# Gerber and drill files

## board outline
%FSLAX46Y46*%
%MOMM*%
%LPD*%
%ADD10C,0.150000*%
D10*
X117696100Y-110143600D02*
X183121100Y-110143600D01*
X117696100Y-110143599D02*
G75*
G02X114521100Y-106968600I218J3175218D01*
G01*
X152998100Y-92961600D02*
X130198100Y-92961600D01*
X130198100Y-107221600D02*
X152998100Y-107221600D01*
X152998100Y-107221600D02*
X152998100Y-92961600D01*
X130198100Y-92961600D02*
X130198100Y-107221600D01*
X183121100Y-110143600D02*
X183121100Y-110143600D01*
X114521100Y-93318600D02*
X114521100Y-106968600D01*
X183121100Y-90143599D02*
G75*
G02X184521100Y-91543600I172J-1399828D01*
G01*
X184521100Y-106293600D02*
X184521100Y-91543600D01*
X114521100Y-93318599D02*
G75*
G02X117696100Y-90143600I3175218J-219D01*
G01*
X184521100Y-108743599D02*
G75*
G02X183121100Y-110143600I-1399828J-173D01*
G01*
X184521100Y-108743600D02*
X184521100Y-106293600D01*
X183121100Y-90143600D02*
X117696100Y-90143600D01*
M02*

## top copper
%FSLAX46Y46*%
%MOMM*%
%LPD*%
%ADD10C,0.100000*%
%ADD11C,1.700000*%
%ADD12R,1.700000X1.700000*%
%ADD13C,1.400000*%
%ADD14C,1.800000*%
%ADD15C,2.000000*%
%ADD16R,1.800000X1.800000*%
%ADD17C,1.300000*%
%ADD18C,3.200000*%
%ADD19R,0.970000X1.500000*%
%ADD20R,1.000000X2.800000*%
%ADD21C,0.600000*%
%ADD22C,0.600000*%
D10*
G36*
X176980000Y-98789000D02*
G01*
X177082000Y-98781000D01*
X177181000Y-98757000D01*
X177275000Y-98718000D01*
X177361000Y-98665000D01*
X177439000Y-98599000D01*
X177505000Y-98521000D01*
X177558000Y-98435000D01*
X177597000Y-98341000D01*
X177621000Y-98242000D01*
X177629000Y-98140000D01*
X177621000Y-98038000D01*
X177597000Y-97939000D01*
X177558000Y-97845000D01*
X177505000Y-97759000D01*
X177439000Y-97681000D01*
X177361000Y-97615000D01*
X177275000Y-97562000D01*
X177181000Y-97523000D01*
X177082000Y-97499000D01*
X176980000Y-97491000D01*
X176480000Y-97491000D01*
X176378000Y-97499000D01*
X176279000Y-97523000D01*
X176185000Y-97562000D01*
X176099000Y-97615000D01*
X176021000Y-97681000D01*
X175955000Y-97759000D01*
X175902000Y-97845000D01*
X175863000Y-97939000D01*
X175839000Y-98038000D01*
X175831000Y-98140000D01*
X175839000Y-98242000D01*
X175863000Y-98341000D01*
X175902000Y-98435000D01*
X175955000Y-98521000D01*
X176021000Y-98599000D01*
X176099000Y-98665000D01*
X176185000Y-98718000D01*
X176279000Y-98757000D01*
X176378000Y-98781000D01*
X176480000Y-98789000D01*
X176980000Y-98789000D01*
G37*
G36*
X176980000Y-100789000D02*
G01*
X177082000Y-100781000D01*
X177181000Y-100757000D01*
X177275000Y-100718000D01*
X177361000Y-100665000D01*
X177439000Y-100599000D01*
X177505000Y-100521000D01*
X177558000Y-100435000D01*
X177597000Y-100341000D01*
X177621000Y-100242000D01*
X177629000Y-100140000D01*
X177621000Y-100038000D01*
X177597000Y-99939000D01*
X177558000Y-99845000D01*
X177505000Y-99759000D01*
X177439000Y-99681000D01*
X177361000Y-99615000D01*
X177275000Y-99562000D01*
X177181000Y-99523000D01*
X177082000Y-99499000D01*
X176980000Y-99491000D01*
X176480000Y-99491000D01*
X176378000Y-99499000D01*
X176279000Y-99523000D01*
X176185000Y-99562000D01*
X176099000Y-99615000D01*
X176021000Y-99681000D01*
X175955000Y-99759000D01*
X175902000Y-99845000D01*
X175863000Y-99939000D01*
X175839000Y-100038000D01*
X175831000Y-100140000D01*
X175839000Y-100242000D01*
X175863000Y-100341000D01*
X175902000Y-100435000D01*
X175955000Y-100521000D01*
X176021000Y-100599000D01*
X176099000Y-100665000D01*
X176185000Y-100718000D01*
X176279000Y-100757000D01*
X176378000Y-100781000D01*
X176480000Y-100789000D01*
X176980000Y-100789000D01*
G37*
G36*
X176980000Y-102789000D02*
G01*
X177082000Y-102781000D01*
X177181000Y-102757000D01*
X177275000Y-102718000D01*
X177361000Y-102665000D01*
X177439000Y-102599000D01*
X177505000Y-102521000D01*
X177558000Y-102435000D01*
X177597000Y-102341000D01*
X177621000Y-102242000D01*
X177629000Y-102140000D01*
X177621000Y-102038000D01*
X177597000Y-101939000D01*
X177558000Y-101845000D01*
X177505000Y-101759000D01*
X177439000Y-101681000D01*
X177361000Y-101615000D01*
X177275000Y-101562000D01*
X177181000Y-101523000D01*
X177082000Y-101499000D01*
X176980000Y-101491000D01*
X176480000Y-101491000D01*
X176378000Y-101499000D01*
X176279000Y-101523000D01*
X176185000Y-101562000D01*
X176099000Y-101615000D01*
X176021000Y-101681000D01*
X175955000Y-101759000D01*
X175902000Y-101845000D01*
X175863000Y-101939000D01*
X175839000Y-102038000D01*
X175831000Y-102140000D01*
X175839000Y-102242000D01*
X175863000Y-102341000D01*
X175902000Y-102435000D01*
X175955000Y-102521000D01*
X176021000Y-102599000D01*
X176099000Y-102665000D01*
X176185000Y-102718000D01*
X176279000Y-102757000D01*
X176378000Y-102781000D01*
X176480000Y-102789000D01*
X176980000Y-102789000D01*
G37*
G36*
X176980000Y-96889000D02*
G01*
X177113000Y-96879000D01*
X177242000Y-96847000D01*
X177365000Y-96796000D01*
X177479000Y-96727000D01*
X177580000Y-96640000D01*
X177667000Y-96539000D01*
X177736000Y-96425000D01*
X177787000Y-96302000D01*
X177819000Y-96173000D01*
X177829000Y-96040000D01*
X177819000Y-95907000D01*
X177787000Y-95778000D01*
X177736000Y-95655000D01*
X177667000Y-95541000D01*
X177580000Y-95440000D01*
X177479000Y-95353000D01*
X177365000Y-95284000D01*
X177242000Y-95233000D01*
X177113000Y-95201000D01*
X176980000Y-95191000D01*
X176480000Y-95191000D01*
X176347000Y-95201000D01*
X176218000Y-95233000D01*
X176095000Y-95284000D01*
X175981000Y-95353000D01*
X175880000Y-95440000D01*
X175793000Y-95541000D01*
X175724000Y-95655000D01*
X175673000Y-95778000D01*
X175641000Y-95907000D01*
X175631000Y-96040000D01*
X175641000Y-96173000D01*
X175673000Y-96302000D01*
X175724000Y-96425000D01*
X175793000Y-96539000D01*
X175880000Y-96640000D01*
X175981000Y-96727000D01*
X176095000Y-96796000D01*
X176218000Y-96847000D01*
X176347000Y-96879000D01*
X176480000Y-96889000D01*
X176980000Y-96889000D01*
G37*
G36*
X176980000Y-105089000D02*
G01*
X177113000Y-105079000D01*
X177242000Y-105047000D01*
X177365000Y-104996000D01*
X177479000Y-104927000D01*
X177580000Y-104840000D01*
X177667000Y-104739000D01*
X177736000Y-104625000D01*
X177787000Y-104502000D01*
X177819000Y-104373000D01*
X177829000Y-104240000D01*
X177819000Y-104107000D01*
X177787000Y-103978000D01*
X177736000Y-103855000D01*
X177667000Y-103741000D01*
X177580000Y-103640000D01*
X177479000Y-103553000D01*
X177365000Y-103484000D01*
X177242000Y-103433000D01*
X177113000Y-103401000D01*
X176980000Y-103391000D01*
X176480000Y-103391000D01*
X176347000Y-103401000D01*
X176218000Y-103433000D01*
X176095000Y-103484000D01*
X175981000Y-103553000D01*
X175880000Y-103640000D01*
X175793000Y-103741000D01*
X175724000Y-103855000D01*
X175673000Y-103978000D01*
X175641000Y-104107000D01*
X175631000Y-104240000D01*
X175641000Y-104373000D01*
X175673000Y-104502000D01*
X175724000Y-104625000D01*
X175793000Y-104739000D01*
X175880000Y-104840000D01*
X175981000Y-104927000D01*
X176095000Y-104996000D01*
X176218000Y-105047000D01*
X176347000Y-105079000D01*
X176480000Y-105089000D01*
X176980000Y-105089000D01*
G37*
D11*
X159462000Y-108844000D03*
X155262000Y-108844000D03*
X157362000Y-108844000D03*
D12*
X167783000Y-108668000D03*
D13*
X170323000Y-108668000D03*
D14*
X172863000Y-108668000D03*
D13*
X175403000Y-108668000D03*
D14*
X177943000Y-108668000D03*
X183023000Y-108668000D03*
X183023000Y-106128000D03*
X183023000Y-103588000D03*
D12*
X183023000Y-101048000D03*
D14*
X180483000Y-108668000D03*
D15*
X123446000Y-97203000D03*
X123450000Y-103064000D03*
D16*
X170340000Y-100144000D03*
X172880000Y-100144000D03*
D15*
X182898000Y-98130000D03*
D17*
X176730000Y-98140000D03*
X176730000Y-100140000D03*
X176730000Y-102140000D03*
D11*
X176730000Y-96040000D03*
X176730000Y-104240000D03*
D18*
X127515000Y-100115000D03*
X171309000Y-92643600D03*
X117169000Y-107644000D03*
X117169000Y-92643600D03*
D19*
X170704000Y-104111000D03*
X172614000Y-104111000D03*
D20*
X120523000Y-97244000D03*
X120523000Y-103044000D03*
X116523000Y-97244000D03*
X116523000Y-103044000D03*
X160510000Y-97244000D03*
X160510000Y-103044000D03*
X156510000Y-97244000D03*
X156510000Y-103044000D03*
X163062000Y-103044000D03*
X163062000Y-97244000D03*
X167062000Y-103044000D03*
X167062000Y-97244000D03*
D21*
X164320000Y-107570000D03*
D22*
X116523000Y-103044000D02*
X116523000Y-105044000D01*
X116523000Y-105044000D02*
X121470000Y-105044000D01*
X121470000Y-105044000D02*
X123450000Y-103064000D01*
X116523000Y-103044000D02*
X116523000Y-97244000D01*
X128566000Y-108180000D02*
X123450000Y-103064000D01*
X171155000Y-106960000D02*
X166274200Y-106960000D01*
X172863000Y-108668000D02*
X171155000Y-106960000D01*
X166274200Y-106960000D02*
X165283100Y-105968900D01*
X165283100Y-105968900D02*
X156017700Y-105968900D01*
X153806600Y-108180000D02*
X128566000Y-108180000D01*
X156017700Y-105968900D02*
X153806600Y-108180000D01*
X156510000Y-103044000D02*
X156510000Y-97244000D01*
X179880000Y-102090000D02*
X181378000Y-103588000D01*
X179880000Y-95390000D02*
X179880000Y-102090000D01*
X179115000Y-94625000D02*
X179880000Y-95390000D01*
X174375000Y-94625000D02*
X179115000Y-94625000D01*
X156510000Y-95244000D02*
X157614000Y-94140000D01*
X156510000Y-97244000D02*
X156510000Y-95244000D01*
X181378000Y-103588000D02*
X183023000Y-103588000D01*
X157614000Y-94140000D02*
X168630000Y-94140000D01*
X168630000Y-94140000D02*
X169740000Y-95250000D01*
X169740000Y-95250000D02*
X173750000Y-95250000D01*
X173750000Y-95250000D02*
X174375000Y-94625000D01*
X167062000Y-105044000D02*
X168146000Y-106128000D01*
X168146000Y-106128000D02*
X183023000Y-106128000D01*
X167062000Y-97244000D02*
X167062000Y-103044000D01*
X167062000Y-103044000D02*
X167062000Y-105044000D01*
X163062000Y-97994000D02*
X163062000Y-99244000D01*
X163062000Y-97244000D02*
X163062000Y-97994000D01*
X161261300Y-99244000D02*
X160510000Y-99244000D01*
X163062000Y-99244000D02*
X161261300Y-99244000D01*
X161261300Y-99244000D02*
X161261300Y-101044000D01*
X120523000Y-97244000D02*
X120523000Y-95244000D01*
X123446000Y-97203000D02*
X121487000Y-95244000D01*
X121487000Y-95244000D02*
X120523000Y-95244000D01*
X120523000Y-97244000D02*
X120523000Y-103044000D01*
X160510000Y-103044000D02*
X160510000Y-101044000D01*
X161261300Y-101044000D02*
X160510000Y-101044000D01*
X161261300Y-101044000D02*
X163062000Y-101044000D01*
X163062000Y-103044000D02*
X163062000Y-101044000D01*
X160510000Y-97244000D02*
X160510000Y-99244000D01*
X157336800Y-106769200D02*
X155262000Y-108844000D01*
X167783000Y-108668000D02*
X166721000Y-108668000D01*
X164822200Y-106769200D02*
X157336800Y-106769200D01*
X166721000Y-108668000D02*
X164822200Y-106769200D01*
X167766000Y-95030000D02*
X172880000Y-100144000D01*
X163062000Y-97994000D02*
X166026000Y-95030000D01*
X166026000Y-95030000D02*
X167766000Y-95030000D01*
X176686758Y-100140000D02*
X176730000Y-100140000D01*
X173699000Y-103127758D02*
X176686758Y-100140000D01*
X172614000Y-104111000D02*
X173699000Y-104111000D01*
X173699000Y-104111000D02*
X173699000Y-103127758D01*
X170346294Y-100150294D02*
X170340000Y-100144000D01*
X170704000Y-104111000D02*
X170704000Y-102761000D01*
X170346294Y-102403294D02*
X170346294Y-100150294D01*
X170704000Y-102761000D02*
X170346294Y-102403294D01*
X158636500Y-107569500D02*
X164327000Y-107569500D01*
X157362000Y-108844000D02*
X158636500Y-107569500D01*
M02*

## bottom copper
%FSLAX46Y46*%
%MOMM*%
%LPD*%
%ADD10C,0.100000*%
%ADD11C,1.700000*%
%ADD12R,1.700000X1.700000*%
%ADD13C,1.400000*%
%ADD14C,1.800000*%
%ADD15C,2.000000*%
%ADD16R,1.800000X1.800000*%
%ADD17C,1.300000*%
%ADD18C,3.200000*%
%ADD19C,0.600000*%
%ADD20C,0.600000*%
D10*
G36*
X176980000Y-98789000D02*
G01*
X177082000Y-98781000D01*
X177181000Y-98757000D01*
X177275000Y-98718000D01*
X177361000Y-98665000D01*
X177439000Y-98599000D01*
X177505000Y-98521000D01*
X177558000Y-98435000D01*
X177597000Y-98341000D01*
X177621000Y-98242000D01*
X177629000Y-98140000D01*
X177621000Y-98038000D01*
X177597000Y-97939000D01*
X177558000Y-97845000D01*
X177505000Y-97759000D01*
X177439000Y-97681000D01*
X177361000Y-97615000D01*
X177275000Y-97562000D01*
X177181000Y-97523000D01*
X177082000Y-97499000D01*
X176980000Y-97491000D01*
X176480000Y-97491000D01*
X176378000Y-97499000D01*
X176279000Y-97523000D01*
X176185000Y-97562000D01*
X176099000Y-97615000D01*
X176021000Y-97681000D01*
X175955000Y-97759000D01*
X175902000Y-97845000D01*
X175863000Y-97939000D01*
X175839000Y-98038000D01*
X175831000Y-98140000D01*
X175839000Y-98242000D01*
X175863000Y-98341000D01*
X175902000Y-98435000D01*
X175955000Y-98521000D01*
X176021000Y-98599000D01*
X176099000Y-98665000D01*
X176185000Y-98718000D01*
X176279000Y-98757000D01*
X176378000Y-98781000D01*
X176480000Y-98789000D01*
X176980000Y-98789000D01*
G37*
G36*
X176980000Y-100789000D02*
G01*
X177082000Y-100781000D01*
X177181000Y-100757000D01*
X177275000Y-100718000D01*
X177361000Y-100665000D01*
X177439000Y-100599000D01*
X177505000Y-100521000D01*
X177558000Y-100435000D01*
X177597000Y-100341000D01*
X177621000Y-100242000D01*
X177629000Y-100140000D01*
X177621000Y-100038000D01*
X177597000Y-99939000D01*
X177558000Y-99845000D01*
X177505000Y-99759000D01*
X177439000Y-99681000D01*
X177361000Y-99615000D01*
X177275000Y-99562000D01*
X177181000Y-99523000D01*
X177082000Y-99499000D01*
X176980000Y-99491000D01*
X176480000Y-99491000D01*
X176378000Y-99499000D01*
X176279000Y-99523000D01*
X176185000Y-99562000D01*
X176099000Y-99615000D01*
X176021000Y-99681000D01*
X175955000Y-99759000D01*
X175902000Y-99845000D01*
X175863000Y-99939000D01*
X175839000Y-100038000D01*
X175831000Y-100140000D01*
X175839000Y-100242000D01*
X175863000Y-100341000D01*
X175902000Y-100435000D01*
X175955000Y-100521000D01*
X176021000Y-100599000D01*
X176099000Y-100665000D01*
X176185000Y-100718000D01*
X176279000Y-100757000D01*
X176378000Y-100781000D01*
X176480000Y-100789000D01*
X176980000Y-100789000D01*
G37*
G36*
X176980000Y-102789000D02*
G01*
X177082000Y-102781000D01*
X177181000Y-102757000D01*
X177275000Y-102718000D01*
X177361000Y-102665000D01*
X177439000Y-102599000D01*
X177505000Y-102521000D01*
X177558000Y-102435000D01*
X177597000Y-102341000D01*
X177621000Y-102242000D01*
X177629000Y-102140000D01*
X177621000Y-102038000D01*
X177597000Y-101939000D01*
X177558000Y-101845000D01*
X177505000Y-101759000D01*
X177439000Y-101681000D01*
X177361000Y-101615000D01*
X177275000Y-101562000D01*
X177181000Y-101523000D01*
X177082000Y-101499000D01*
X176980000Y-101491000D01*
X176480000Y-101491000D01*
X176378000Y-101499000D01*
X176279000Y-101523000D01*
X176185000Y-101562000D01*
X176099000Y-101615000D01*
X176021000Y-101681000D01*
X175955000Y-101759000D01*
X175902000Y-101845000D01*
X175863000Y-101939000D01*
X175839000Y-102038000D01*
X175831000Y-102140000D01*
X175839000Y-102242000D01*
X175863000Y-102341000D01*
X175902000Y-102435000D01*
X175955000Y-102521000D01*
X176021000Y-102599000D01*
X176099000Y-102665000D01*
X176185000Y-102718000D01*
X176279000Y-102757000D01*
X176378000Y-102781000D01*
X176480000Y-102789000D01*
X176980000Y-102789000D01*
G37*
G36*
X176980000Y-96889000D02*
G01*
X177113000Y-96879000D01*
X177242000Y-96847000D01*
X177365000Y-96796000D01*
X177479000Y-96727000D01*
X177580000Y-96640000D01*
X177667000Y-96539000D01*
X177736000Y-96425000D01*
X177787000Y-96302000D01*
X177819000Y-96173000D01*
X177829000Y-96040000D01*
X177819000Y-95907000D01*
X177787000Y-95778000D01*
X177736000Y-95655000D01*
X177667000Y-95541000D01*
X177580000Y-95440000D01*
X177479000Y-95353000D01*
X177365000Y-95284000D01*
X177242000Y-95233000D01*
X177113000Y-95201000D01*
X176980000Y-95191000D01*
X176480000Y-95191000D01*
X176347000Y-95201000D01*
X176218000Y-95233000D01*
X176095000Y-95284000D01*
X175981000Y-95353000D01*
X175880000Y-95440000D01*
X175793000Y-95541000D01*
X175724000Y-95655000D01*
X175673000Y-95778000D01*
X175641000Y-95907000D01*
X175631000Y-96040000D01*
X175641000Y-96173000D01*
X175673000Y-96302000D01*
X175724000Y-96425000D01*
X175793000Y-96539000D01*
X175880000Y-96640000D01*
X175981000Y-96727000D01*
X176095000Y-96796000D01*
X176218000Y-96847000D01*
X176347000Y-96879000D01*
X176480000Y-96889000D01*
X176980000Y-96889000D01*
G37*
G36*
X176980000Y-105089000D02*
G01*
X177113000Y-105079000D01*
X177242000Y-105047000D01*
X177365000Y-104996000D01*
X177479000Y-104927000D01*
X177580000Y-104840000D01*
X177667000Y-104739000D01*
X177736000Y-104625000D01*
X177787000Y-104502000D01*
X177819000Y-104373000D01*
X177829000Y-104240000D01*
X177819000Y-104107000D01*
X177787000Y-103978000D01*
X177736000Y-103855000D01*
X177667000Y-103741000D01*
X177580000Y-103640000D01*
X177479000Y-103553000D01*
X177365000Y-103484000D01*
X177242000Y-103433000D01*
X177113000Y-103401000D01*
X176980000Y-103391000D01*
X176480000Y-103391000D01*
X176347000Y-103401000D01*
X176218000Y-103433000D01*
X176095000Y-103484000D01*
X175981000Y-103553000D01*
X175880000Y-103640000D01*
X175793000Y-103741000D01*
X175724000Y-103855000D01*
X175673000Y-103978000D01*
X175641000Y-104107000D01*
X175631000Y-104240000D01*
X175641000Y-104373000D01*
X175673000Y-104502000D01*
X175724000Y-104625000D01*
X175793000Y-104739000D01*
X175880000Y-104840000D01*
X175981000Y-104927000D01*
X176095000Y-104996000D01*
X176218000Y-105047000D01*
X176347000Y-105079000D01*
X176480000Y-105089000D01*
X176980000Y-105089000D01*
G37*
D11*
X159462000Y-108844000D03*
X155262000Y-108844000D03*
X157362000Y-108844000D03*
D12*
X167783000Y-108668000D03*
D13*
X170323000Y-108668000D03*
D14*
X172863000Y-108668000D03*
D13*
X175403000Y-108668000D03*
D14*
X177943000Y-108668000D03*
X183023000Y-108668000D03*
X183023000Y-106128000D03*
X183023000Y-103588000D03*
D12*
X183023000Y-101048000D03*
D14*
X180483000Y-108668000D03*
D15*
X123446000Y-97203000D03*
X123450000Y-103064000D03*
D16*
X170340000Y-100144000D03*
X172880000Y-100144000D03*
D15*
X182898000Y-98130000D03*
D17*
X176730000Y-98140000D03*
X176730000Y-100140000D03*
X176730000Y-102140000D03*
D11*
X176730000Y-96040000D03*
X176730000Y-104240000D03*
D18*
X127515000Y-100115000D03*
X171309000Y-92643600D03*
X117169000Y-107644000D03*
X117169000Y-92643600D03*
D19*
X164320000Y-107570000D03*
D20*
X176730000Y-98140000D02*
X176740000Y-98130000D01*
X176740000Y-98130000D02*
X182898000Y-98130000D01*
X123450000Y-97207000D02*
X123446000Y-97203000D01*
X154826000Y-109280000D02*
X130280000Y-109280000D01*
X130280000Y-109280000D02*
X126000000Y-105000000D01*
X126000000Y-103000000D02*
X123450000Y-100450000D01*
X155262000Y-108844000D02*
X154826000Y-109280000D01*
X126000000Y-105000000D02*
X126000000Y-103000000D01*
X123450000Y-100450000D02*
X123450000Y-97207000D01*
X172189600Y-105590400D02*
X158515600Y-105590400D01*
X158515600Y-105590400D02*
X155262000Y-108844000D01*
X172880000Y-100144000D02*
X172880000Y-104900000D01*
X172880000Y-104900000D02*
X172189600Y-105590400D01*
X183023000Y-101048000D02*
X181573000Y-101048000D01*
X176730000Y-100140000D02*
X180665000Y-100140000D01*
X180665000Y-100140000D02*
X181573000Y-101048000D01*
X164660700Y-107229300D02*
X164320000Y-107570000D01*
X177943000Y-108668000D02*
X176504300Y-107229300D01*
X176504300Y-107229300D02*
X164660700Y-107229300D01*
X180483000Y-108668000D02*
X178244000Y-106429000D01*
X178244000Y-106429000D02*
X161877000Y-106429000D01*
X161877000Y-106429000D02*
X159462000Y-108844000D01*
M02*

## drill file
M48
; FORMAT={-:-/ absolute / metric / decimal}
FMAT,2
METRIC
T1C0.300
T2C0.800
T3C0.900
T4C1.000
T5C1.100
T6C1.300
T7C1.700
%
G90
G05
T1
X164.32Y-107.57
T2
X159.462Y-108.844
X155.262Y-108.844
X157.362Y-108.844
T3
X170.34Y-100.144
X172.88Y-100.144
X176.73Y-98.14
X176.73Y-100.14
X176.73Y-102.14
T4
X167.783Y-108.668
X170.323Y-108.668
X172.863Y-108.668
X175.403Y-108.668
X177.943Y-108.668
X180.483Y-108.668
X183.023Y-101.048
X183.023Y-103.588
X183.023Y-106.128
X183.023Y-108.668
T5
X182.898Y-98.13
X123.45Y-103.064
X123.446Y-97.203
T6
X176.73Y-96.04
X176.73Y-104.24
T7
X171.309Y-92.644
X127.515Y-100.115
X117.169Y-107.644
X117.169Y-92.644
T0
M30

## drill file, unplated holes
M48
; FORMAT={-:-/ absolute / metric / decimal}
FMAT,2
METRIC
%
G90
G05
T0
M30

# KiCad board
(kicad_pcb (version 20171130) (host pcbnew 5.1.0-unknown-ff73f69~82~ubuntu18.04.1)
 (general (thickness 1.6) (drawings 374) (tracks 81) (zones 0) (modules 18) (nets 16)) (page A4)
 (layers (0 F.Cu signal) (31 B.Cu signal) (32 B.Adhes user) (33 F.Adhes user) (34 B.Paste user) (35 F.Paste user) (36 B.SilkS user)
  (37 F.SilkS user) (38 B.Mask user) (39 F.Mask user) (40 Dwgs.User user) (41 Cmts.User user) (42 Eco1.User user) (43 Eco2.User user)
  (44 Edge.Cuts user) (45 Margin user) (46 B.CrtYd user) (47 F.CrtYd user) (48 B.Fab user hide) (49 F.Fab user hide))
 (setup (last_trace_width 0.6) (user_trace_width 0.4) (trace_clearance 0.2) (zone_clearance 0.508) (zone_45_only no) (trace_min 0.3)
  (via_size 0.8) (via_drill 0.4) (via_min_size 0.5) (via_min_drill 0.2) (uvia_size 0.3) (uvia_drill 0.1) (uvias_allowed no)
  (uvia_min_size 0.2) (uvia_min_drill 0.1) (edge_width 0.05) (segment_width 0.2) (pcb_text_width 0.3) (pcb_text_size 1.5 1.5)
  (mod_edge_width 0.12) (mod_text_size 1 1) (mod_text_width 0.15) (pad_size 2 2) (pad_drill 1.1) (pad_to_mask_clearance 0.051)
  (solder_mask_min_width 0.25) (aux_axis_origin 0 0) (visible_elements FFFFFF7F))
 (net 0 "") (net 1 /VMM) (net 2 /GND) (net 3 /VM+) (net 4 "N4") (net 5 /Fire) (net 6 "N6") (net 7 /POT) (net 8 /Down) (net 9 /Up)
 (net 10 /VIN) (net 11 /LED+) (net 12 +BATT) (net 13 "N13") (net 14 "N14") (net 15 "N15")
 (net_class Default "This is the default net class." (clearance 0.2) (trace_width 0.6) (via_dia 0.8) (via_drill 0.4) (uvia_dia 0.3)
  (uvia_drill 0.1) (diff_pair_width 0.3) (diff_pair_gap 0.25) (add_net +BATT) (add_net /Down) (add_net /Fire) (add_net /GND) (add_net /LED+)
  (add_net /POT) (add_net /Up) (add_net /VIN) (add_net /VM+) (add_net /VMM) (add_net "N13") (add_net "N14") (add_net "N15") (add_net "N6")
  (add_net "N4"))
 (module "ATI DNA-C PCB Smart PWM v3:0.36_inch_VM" (layer F.Cu) (at 141.72 100.27)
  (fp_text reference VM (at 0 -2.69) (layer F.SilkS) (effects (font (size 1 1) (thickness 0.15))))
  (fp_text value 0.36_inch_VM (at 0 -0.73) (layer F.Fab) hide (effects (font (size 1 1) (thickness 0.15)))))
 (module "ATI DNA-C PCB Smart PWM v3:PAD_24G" (layer F.Cu) (at 159.462 108.844)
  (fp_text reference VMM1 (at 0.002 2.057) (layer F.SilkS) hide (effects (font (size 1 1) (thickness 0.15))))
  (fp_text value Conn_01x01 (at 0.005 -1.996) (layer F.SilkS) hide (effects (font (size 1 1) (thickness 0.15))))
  (pad 1 thru_hole circle (at 0 0 90) (size 1.7 1.7) (drill 0.8) (layers *.Cu *.Mask) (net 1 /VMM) (solder_mask_margin 0.1016)
   (zone_connect 2)))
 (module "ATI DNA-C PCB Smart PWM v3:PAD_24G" (layer F.Cu) (at 155.262 108.844)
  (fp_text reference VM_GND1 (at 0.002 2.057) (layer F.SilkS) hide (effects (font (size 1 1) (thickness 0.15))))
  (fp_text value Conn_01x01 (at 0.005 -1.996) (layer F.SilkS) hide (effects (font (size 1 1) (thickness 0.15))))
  (pad 1 thru_hole circle (at 0 0 90) (size 1.7 1.7) (drill 0.8) (layers *.Cu *.Mask) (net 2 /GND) (solder_mask_margin 0.1016)
   (zone_connect 2)))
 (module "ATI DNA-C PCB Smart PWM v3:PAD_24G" (layer F.Cu) (at 157.362 108.844)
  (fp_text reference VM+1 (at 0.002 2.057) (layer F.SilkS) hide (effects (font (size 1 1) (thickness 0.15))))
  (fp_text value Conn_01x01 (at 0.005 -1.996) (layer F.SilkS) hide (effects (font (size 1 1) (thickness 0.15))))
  (pad 1 thru_hole circle (at 0 0 90) (size 1.7 1.7) (drill 0.8) (layers *.Cu *.Mask) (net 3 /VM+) (solder_mask_margin 0.1016)
   (zone_connect 2)))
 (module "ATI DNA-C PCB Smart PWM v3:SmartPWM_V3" (layer F.Cu) (at 175.438 104.848)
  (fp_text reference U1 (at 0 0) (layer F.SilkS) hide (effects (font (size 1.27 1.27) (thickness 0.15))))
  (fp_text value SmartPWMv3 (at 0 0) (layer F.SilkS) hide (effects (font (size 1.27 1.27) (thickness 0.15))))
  (pad 10 thru_hole rect (at -7.655 3.82) (size 1.7 1.7) (drill 1) (layers *.Cu *.Mask) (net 2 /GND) (zone_connect 2))
  (pad 9 thru_hole circle (at -5.115 3.82) (size 1.4 1.4) (drill 1) (layers *.Cu *.Mask) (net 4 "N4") (zone_connect 2))
  (pad 8 thru_hole circle (at -2.575 3.82) (size 1.8 1.8) (drill 1) (layers *.Cu *.Mask) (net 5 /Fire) (zone_connect 2))
  (pad 7 thru_hole circle (at -0.035 3.82) (size 1.4 1.4) (drill 1) (layers *.Cu *.Mask) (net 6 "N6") (zone_connect 2))
  (pad 6 thru_hole circle (at 2.505 3.82) (size 1.8 1.8) (drill 1) (layers *.Cu *.Mask) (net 3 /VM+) (zone_connect 2))
  (pad 4 thru_hole circle (at 7.585 3.82) (size 1.8 1.8) (drill 1) (layers *.Cu *.Mask) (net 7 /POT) (zone_connect 2))
  (pad 3 thru_hole circle (at 7.585 1.28) (size 1.8 1.8) (drill 1) (layers *.Cu *.Mask) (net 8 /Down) (zone_connect 2))
  (pad 2 thru_hole circle (at 7.585 -1.26) (size 1.8 1.8) (drill 1) (layers *.Cu *.Mask) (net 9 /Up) (zone_connect 2))
  (pad 1 thru_hole rect (at 7.585 -3.8 90) (size 1.7 1.7) (drill 1) (layers *.Cu *.Mask) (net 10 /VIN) (zone_connect 2))
  (pad 5 thru_hole circle (at 5.045 3.82) (size 1.8 1.8) (drill 1) (layers *.Cu *.Mask) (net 1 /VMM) (zone_connect 2)))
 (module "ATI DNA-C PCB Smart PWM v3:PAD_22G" (layer F.Cu) (at 123.446 97.203)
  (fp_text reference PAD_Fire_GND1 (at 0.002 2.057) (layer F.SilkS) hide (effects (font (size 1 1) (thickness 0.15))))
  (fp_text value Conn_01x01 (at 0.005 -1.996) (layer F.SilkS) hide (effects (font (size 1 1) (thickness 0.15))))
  (pad 1 thru_hole circle (at 0 0 90) (size 2 2) (drill 1.1) (layers *.Cu *.Mask) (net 2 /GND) (solder_mask_margin 0.1016) (zone_connect 2)))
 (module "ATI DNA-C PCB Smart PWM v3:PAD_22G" (layer F.Cu) (at 123.45 103.064)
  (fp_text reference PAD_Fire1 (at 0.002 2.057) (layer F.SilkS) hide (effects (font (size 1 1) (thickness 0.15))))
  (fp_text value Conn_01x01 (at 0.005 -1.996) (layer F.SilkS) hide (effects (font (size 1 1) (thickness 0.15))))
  (pad 1 thru_hole circle (at 0 0 90) (size 2 2) (drill 1.1) (layers *.Cu *.Mask) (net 5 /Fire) (solder_mask_margin 0.1016) (zone_connect 2)))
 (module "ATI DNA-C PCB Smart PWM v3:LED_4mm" (layer F.Cu) (at 171.62 100.144 180)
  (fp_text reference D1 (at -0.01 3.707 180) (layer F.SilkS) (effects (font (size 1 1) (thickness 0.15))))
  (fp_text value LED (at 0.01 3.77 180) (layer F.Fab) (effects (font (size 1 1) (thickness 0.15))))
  (pad 2 thru_hole rect (at 1.28 0 180) (size 1.8 1.8) (drill 0.9) (layers *.Cu *.Mask) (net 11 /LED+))
  (pad 1 thru_hole rect (at -1.26 0 180) (size 1.8 1.8) (drill 0.9) (layers *.Cu *.Mask) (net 2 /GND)))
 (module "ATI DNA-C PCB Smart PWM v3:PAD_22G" (layer F.Cu) (at 182.898 98.13)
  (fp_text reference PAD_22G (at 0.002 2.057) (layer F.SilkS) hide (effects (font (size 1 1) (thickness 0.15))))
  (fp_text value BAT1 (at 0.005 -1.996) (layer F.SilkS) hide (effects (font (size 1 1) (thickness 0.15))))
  (pad 1 thru_hole circle (at 0 0 90) (size 2 2) (drill 1.1) (layers *.Cu *.Mask) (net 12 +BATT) (solder_mask_margin 0.1016)
   (zone_connect 2)))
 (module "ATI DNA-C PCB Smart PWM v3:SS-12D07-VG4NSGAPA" (layer F.Cu) (at 176.73 100.14 270)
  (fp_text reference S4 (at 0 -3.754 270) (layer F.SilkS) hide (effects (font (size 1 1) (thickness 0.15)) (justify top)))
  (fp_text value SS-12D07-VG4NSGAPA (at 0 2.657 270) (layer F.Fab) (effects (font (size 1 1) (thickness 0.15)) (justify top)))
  (fp_poly
   (pts (xy -1.351 -0.25) (xy -1.359 -0.352) (xy -1.383 -0.451) (xy -1.422 -0.545) (xy -1.475 -0.631) (xy -1.541 -0.709) (xy -1.619 -0.775)
    (xy -1.705 -0.828) (xy -1.799 -0.867) (xy -1.898 -0.891) (xy -2 -0.899) (xy -2.102 -0.891) (xy -2.201 -0.867) (xy -2.295 -0.828)
    (xy -2.381 -0.775) (xy -2.459 -0.709) (xy -2.525 -0.631) (xy -2.578 -0.545) (xy -2.617 -0.451) (xy -2.641 -0.352) (xy -2.649 -0.25)
    (xy -2.649 0.25) (xy -2.641 0.352) (xy -2.617 0.451) (xy -2.578 0.545) (xy -2.525 0.631) (xy -2.459 0.709) (xy -2.381 0.775)
    (xy -2.295 0.828) (xy -2.201 0.867) (xy -2.102 0.891) (xy -2 0.899) (xy -1.898 0.891) (xy -1.799 0.867) (xy -1.705 0.828)
    (xy -1.619 0.775) (xy -1.541 0.709) (xy -1.475 0.631) (xy -1.422 0.545) (xy -1.383 0.451) (xy -1.359 0.352) (xy -1.351 0.25))
   (layer F.Cu) (width 0))
  (fp_poly
   (pts (xy -1.351 -0.25) (xy -1.359 -0.352) (xy -1.383 -0.451) (xy -1.422 -0.545) (xy -1.475 -0.631) (xy -1.541 -0.709) (xy -1.619 -0.775)
    (xy -1.705 -0.828) (xy -1.799 -0.867) (xy -1.898 -0.891) (xy -2 -0.899) (xy -2.102 -0.891) (xy -2.201 -0.867) (xy -2.295 -0.828)
    (xy -2.381 -0.775) (xy -2.459 -0.709) (xy -2.525 -0.631) (xy -2.578 -0.545) (xy -2.617 -0.451) (xy -2.641 -0.352) (xy -2.649 -0.25)
    (xy -2.649 0.25) (xy -2.641 0.352) (xy -2.617 0.451) (xy -2.578 0.545) (xy -2.525 0.631) (xy -2.459 0.709) (xy -2.381 0.775)
    (xy -2.295 0.828) (xy -2.201 0.867) (xy -2.102 0.891) (xy -2 0.899) (xy -1.898 0.891) (xy -1.799 0.867) (xy -1.705 0.828)
    (xy -1.619 0.775) (xy -1.541 0.709) (xy -1.475 0.631) (xy -1.422 0.545) (xy -1.383 0.451) (xy -1.359 0.352) (xy -1.351 0.25))
   (layer B.Cu) (width 0))
  (fp_poly
   (pts (xy 0.649 -0.25) (xy 0.641 -0.352) (xy 0.617 -0.451) (xy 0.578 -0.545) (xy 0.525 -0.631) (xy 0.459 -0.709) (xy 0.381 -0.775)
    (xy 0.295 -0.828) (xy 0.201 -0.867) (xy 0.102 -0.891) (xy 0 -0.899) (xy -0.102 -0.891) (xy -0.201 -0.867) (xy -0.295 -0.828)
    (xy -0.381 -0.775) (xy -0.459 -0.709) (xy -0.525 -0.631) (xy -0.578 -0.545) (xy -0.617 -0.451) (xy -0.641 -0.352) (xy -0.649 -0.25)
    (xy -0.649 0.25) (xy -0.641 0.352) (xy -0.617 0.451) (xy -0.578 0.545) (xy -0.525 0.631) (xy -0.459 0.709) (xy -0.381 0.775)
    (xy -0.295 0.828) (xy -0.201 0.867) (xy -0.102 0.891) (xy 0 0.899) (xy 0.102 0.891) (xy 0.201 0.867) (xy 0.295 0.828) (xy 0.381 0.775)
    (xy 0.459 0.709) (xy 0.525 0.631) (xy 0.578 0.545) (xy 0.617 0.451) (xy 0.641 0.352) (xy 0.649 0.25))
   (layer F.Cu) (width 0))
  (fp_poly
   (pts (xy 0.649 -0.25) (xy 0.641 -0.352) (xy 0.617 -0.451) (xy 0.578 -0.545) (xy 0.525 -0.631) (xy 0.459 -0.709) (xy 0.381 -0.775)
    (xy 0.295 -0.828) (xy 0.201 -0.867) (xy 0.102 -0.891) (xy 0 -0.899) (xy -0.102 -0.891) (xy -0.201 -0.867) (xy -0.295 -0.828)
    (xy -0.381 -0.775) (xy -0.459 -0.709) (xy -0.525 -0.631) (xy -0.578 -0.545) (xy -0.617 -0.451) (xy -0.641 -0.352) (xy -0.649 -0.25)
    (xy -0.649 0.25) (xy -0.641 0.352) (xy -0.617 0.451) (xy -0.578 0.545) (xy -0.525 0.631) (xy -0.459 0.709) (xy -0.381 0.775)
    (xy -0.295 0.828) (xy -0.201 0.867) (xy -0.102 0.891) (xy 0 0.899) (xy 0.102 0.891) (xy 0.201 0.867) (xy 0.295 0.828) (xy 0.381 0.775)
    (xy 0.459 0.709) (xy 0.525 0.631) (xy 0.578 0.545) (xy 0.617 0.451) (xy 0.641 0.352) (xy 0.649 0.25))
   (layer B.Cu) (width 0))
  (fp_poly
   (pts (xy 2.649 -0.25) (xy 2.641 -0.352) (xy 2.617 -0.451) (xy 2.578 -0.545) (xy 2.525 -0.631) (xy 2.459 -0.709) (xy 2.381 -0.775)
    (xy 2.295 -0.828) (xy 2.201 -0.867) (xy 2.102 -0.891) (xy 2 -0.899) (xy 1.898 -0.891) (xy 1.799 -0.867) (xy 1.705 -0.828)
    (xy 1.619 -0.775) (xy 1.541 -0.709) (xy 1.475 -0.631) (xy 1.422 -0.545) (xy 1.383 -0.451) (xy 1.359 -0.352) (xy 1.351 -0.25)
    (xy 1.351 0.25) (xy 1.359 0.352) (xy 1.383 0.451) (xy 1.422 0.545) (xy 1.475 0.631) (xy 1.541 0.709) (xy 1.619 0.775) (xy 1.705 0.828)
    (xy 1.799 0.867) (xy 1.898 0.891) (xy 2 0.899) (xy 2.102 0.891) (xy 2.201 0.867) (xy 2.295 0.828) (xy 2.381 0.775) (xy 2.459 0.709)
    (xy 2.525 0.631) (xy 2.578 0.545) (xy 2.617 0.451) (xy 2.641 0.352) (xy 2.649 0.25))
   (layer F.Cu) (width 0))
  (fp_poly
   (pts (xy 2.649 -0.25) (xy 2.641 -0.352) (xy 2.617 -0.451) (xy 2.578 -0.545) (xy 2.525 -0.631) (xy 2.459 -0.709) (xy 2.381 -0.775)
    (xy 2.295 -0.828) (xy 2.201 -0.867) (xy 2.102 -0.891) (xy 2 -0.899) (xy 1.898 -0.891) (xy 1.799 -0.867) (xy 1.705 -0.828)
    (xy 1.619 -0.775) (xy 1.541 -0.709) (xy 1.475 -0.631) (xy 1.422 -0.545) (xy 1.383 -0.451) (xy 1.359 -0.352) (xy 1.351 -0.25)
    (xy 1.351 0.25) (xy 1.359 0.352) (xy 1.383 0.451) (xy 1.422 0.545) (xy 1.475 0.631) (xy 1.541 0.709) (xy 1.619 0.775) (xy 1.705 0.828)
    (xy 1.799 0.867) (xy 1.898 0.891) (xy 2 0.899) (xy 2.102 0.891) (xy 2.201 0.867) (xy 2.295 0.828) (xy 2.381 0.775) (xy 2.459 0.709)
    (xy 2.525 0.631) (xy 2.578 0.545) (xy 2.617 0.451) (xy 2.641 0.352) (xy 2.649 0.25))
   (layer B.Cu) (width 0))
  (fp_poly
   (pts (xy -3.251 -0.25) (xy -3.261 -0.383) (xy -3.293 -0.512) (xy -3.344 -0.635) (xy -3.413 -0.749) (xy -3.5 -0.85) (xy -3.601 -0.937)
    (xy -3.715 -1.006) (xy -3.838 -1.057) (xy -3.967 -1.089) (xy -4.1 -1.099) (xy -4.233 -1.089) (xy -4.362 -1.057) (xy -4.485 -1.006)
    (xy -4.599 -0.937) (xy -4.7 -0.85) (xy -4.787 -0.749) (xy -4.856 -0.635) (xy -4.907 -0.512) (xy -4.939 -0.383) (xy -4.949 -0.25)
    (xy -4.949 0.25) (xy -4.939 0.383) (xy -4.907 0.512) (xy -4.856 0.635) (xy -4.787 0.749) (xy -4.7 0.85) (xy -4.599 0.937)
    (xy -4.485 1.006) (xy -4.362 1.057) (xy -4.233 1.089) (xy -4.1 1.099) (xy -3.967 1.089) (xy -3.838 1.057) (xy -3.715 1.006)
    (xy -3.601 0.937) (xy -3.5 0.85) (xy -3.413 0.749) (xy -3.344 0.635) (xy -3.293 0.512) (xy -3.261 0.383) (xy -3.251 0.25))
   (layer F.Cu) (width 0))
  (fp_poly
   (pts (xy -3.251 -0.25) (xy -3.261 -0.383) (xy -3.293 -0.512) (xy -3.344 -0.635) (xy -3.413 -0.749) (xy -3.5 -0.85) (xy -3.601 -0.937)
    (xy -3.715 -1.006) (xy -3.838 -1.057) (xy -3.967 -1.089) (xy -4.1 -1.099) (xy -4.233 -1.089) (xy -4.362 -1.057) (xy -4.485 -1.006)
    (xy -4.599 -0.937) (xy -4.7 -0.85) (xy -4.787 -0.749) (xy -4.856 -0.635) (xy -4.907 -0.512) (xy -4.939 -0.383) (xy -4.949 -0.25)
    (xy -4.949 0.25) (xy -4.939 0.383) (xy -4.907 0.512) (xy -4.856 0.635) (xy -4.787 0.749) (xy -4.7 0.85) (xy -4.599 0.937)
    (xy -4.485 1.006) (xy -4.362 1.057) (xy -4.233 1.089) (xy -4.1 1.099) (xy -3.967 1.089) (xy -3.838 1.057) (xy -3.715 1.006)
    (xy -3.601 0.937) (xy -3.5 0.85) (xy -3.413 0.749) (xy -3.344 0.635) (xy -3.293 0.512) (xy -3.261 0.383) (xy -3.251 0.25))
   (layer B.Cu) (width 0))
  (fp_poly
   (pts (xy 4.949 -0.25) (xy 4.939 -0.383) (xy 4.907 -0.512) (xy 4.856 -0.635) (xy 4.787 -0.749) (xy 4.7 -0.85) (xy 4.599 -0.937)
    (xy 4.485 -1.006) (xy 4.362 -1.057) (xy 4.233 -1.089) (xy 4.1 -1.099) (xy 3.967 -1.089) (xy 3.838 -1.057) (xy 3.715 -1.006)
    (xy 3.601 -0.937) (xy 3.5 -0.85) (xy 3.413 -0.749) (xy 3.344 -0.635) (xy 3.293 -0.512) (xy 3.261 -0.383) (xy 3.251 -0.25)
    (xy 3.251 0.25) (xy 3.261 0.383) (xy 3.293 0.512) (xy 3.344 0.635) (xy 3.413 0.749) (xy 3.5 0.85) (xy 3.601 0.937) (xy 3.715 1.006)
    (xy 3.838 1.057) (xy 3.967 1.089) (xy 4.1 1.099) (xy 4.233 1.089) (xy 4.362 1.057) (xy 4.485 1.006) (xy 4.599 0.937) (xy 4.7 0.85)
    (xy 4.787 0.749) (xy 4.856 0.635) (xy 4.907 0.512) (xy 4.939 0.383) (xy 4.949 0.25))
   (layer F.Cu) (width 0))
  (fp_poly
   (pts (xy 4.949 -0.25) (xy 4.939 -0.383) (xy 4.907 -0.512) (xy 4.856 -0.635) (xy 4.787 -0.749) (xy 4.7 -0.85) (xy 4.599 -0.937)
    (xy 4.485 -1.006) (xy 4.362 -1.057) (xy 4.233 -1.089) (xy 4.1 -1.099) (xy 3.967 -1.089) (xy 3.838 -1.057) (xy 3.715 -1.006)
    (xy 3.601 -0.937) (xy 3.5 -0.85) (xy 3.413 -0.749) (xy 3.344 -0.635) (xy 3.293 -0.512) (xy 3.261 -0.383) (xy 3.251 -0.25)
    (xy 3.251 0.25) (xy 3.261 0.383) (xy 3.293 0.512) (xy 3.344 0.635) (xy 3.413 0.749) (xy 3.5 0.85) (xy 3.601 0.937) (xy 3.715 1.006)
    (xy 3.838 1.057) (xy 3.967 1.089) (xy 4.1 1.099) (xy 4.233 1.089) (xy 4.362 1.057) (xy 4.485 1.006) (xy 4.599 0.937) (xy 4.7 0.85)
    (xy 4.787 0.749) (xy 4.856 0.635) (xy 4.907 0.512) (xy 4.939 0.383) (xy 4.949 0.25))
   (layer B.Cu) (width 0))
  (pad 1 thru_hole circle (at -2 0) (size 1.3 1.3) (drill 0.9) (layers *.Cu *.Mask) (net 12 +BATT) (solder_mask_margin 0.1016)
   (zone_connect 2))
  (pad 2 thru_hole circle (at 0 0) (size 1.3 1.3) (drill 0.9) (layers *.Cu *.Mask) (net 10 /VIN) (solder_mask_margin 0.1016)
   (zone_connect 2))
  (pad 3 thru_hole circle (at 2 0) (size 1.3 1.3) (drill 0.9) (layers *.Cu *.Mask) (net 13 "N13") (solder_mask_margin 0.1016)
   (zone_connect 2))
  (pad MH1 thru_hole circle (at -4.1 0) (size 1.7 1.7) (drill 1.3) (layers *.Cu *.Mask) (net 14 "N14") (solder_mask_margin 0.1016)
   (zone_connect 2))
  (pad MH2 thru_hole circle (at 4.1 0) (size 1.7 1.7) (drill 1.3) (layers *.Cu *.Mask) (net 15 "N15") (solder_mask_margin 0.1016)
   (zone_connect 2)))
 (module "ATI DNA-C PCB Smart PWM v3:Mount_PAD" (layer F.Cu) (at 127.515 100.115 90)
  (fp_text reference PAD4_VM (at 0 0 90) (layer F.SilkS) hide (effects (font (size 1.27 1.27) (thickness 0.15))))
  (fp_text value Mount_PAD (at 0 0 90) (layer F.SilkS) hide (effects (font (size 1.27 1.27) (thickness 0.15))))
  (pad 1 thru_hole circle (at 0 0 90) (size 3.2 3.2) (drill 1.7) (layers *.Cu *.Mask) (zone_connect 2)))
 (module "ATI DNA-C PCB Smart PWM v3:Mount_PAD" (layer F.Cu) (at 171.309 92.6436 90)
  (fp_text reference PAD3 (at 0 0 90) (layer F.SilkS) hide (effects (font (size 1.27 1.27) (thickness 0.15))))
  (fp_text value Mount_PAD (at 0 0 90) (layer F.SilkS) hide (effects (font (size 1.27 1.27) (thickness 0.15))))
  (pad 1 thru_hole circle (at 0 0 90) (size 3.2 3.2) (drill 1.7) (layers *.Cu *.Mask) (zone_connect 2)))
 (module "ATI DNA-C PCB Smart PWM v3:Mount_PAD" (layer F.Cu) (at 117.169 107.644 90)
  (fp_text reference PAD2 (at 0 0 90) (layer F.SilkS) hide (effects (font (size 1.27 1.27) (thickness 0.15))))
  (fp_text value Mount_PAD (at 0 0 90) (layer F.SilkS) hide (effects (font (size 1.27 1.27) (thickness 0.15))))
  (pad 1 thru_hole circle (at 0 0 90) (size 3.2 3.2) (drill 1.7) (layers *.Cu *.Mask) (zone_connect 2)))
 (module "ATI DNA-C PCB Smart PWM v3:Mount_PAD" (layer F.Cu) (at 117.169 92.6436 90)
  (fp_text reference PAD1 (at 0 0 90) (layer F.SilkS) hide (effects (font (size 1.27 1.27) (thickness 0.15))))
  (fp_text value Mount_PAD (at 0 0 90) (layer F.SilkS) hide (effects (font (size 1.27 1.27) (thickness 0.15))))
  (pad 1 thru_hole circle (at 0 0 90) (size 3.2 3.2) (drill 1.7) (layers *.Cu *.Mask) (zone_connect 2)))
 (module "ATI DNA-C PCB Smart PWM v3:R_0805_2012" (layer F.Cu) (at 171.659 104.111 180)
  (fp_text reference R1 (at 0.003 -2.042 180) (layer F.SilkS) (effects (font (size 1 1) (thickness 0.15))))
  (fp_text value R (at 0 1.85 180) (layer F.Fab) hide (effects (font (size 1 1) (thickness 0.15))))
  (pad 2 smd rect (at 0.955 0 180) (size 0.97 1.5) (layers F.Cu F.Paste F.Mask) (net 11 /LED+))
  (pad 1 smd rect (at -0.955 0 180) (size 0.97 1.5) (layers F.Cu F.Paste F.Mask) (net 10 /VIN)))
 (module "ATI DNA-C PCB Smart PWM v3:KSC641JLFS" (layer F.Cu) (at 118.523 100.144 270)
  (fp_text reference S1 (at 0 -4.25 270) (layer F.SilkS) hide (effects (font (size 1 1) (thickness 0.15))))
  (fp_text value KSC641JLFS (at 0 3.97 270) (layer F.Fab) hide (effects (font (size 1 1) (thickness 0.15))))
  (pad 1 smd rect (at -2.9 -2 270) (size 2.8 1) (layers F.Cu F.Paste F.Mask) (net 2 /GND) (solder_paste_margin -0.1016) (zone_connect 2))
  (pad 2 smd rect (at 2.9 -2 270) (size 2.8 1) (layers F.Cu F.Paste F.Mask) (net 2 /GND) (solder_paste_margin -0.1016) (zone_connect 2))
  (pad 3 smd rect (at -2.9 2 270) (size 2.8 1) (layers F.Cu F.Paste F.Mask) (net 5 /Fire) (solder_paste_margin -0.1016) (zone_connect 2))
  (pad 4 smd rect (at 2.9 2 270) (size 2.8 1) (layers F.Cu F.Paste F.Mask) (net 5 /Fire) (solder_paste_margin -0.1016) (zone_connect 2)))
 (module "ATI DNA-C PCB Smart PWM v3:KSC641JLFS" (layer F.Cu) (at 158.51 100.144 270)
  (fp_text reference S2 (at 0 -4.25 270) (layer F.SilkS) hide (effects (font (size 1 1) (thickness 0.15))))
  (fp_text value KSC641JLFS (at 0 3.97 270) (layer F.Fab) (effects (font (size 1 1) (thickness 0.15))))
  (pad 1 smd rect (at -2.9 -2 270) (size 2.8 1) (layers F.Cu F.Paste F.Mask) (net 2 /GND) (solder_paste_margin -0.1016) (zone_connect 2))
  (pad 2 smd rect (at 2.9 -2 270) (size 2.8 1) (layers F.Cu F.Paste F.Mask) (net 2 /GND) (solder_paste_margin -0.1016) (zone_connect 2))
  (pad 3 smd rect (at -2.9 2 270) (size 2.8 1) (layers F.Cu F.Paste F.Mask) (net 9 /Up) (solder_paste_margin -0.1016) (zone_connect 2))
  (pad 4 smd rect (at 2.9 2 270) (size 2.8 1) (layers F.Cu F.Paste F.Mask) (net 9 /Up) (solder_paste_margin -0.1016) (zone_connect 2)))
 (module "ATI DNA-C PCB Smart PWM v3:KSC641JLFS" (layer F.Cu) (at 165.062 100.144 90)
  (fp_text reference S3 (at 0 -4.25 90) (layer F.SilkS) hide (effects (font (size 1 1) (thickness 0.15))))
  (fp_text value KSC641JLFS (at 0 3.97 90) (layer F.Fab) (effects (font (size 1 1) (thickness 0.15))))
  (pad 1 smd rect (at -2.9 -2 90) (size 2.8 1) (layers F.Cu F.Paste F.Mask) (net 2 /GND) (solder_paste_margin -0.1016) (zone_connect 2))
  (pad 2 smd rect (at 2.9 -2 90) (size 2.8 1) (layers F.Cu F.Paste F.Mask) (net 2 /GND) (solder_paste_margin -0.1016) (zone_connect 2))
  (pad 3 smd rect (at -2.9 2 90) (size 2.8 1) (layers F.Cu F.Paste F.Mask) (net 8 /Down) (solder_paste_margin -0.1016) (zone_connect 2))
  (pad 4 smd rect (at 2.9 2 90) (size 2.8 1) (layers F.Cu F.Paste F.Mask) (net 8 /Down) (solder_paste_margin -0.1016) (zone_connect 2)))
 (gr_line (start 117.6961 110.1436) (end 183.1211 110.1436) (layer Edge.Cuts) (width 0.15))
 (gr_arc (start 117.696318 106.968381) (end 114.5211 106.9686) (angle -89.99211) (layer Edge.Cuts) (width 0.15))
 (gr_line (start 152.9981 92.9616) (end 130.1981 92.9616) (layer Edge.Cuts) (width 0.15))
 (gr_line (start 130.1981 107.2216) (end 152.9981 107.2216) (layer Edge.Cuts) (width 0.15))
 (gr_line (start 152.9981 107.2216) (end 152.9981 92.9616) (layer Edge.Cuts) (width 0.15))
 (gr_line (start 130.1981 92.9616) (end 130.1981 107.2216) (layer Edge.Cuts) (width 0.15))
 (gr_line (start 183.1211 110.1436) (end 183.1211 110.1436) (layer Edge.Cuts) (width 0.15))
 (gr_line (start 114.5211 93.3186) (end 114.5211 106.9686) (layer Edge.Cuts) (width 0.15))
 (gr_arc (start 183.121272 91.543427) (end 184.5211 91.5436) (angle -90.014114) (layer Edge.Cuts) (width 0.15))
 (gr_line (start 184.5211 106.2936) (end 184.5211 91.5436) (layer Edge.Cuts) (width 0.15))
 (gr_arc (start 117.696318 93.318818) (end 117.6961 90.1436) (angle -89.99211) (layer Edge.Cuts) (width 0.15))
 (gr_arc (start 183.121272 108.743772) (end 183.1211 110.1436) (angle -90.014114) (layer Edge.Cuts) (width 0.15))
 (gr_line (start 184.5211 108.7436) (end 184.5211 106.2936) (layer Edge.Cuts) (width 0.15))
 (gr_line (start 183.1211 90.1436) (end 117.6961 90.1436) (layer Edge.Cuts) (width 0.15))
 (segment (start 116.523 103.044) (end 116.523 105.044) (width 0.6) (layer F.Cu) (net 5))
 (segment (start 116.523 105.044) (end 121.47 105.044) (width 0.6) (layer F.Cu) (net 5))
 (segment (start 121.47 105.044) (end 123.45 103.064) (width 0.6) (layer F.Cu) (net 5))
 (segment (start 116.523 103.044) (end 116.523 97.244) (width 0.6) (layer F.Cu) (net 5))
 (segment (start 128.566 108.18) (end 123.45 103.064) (width 0.6) (layer F.Cu) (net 5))
 (segment (start 171.155 106.96) (end 166.2742 106.96) (width 0.6) (layer F.Cu) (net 5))
 (segment (start 172.863 108.668) (end 171.155 106.96) (width 0.6) (layer F.Cu) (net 5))
 (segment (start 166.2742 106.96) (end 165.2831 105.9689) (width 0.6) (layer F.Cu) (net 5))
 (segment (start 165.2831 105.9689) (end 156.0177 105.9689) (width 0.6) (layer F.Cu) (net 5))
 (segment (start 153.8066 108.18) (end 128.566 108.18) (width 0.6) (layer F.Cu) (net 5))
 (segment (start 156.0177 105.9689) (end 153.8066 108.18) (width 0.6) (layer F.Cu) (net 5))
 (segment (start 156.51 103.044) (end 156.51 97.244) (width 0.6) (layer F.Cu) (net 9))
 (segment (start 179.88 102.09) (end 181.378 103.588) (width 0.6) (layer F.Cu) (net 9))
 (segment (start 179.88 95.39) (end 179.88 102.09) (width 0.6) (layer F.Cu) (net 9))
 (segment (start 179.115 94.625) (end 179.88 95.39) (width 0.6) (layer F.Cu) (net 9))
 (segment (start 174.375 94.625) (end 179.115 94.625) (width 0.6) (layer F.Cu) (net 9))
 (segment (start 156.51 95.244) (end 157.614 94.14) (width 0.6) (layer F.Cu) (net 9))
 (segment (start 156.51 97.244) (end 156.51 95.244) (width 0.6) (layer F.Cu) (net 9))
 (segment (start 181.378 103.588) (end 183.023 103.588) (width 0.6) (layer F.Cu) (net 9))
 (segment (start 157.614 94.14) (end 168.63 94.14) (width 0.6) (layer F.Cu) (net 9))
 (segment (start 168.63 94.14) (end 169.74 95.25) (width 0.6) (layer F.Cu) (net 9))
 (segment (start 169.74 95.25) (end 173.75 95.25) (width 0.6) (layer F.Cu) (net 9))
 (segment (start 173.75 95.25) (end 174.375 94.625) (width 0.6) (layer F.Cu) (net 9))
 (segment (start 167.062 105.044) (end 168.146 106.128) (width 0.6) (layer F.Cu) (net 8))
 (segment (start 168.146 106.128) (end 183.023 106.128) (width 0.6) (layer F.Cu) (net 8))
 (segment (start 167.062 97.244) (end 167.062 103.044) (width 0.6) (layer F.Cu) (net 8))
 (segment (start 167.062 103.044) (end 167.062 105.044) (width 0.6) (layer F.Cu) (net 8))
 (segment (start 176.73 98.14) (end 176.74 98.13) (width 0.6) (layer B.Cu) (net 12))
 (segment (start 176.74 98.13) (end 182.898 98.13) (width 0.6) (layer B.Cu) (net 12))
 (segment (start 163.062 97.994) (end 163.062 99.244) (width 0.6) (layer F.Cu) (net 2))
 (segment (start 163.062 97.244) (end 163.062 97.994) (width 0.6) (layer F.Cu) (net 2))
 (segment (start 161.2613 99.244) (end 160.51 99.244) (width 0.6) (layer F.Cu) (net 2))
 (segment (start 163.062 99.244) (end 161.2613 99.244) (width 0.6) (layer F.Cu) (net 2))
 (segment (start 161.2613 99.244) (end 161.2613 101.044) (width 0.6) (layer F.Cu) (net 2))
 (segment (start 120.523 97.244) (end 120.523 95.244) (width 0.6) (layer F.Cu) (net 2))
 (segment (start 123.446 97.203) (end 121.487 95.244) (width 0.6) (layer F.Cu) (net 2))
 (segment (start 121.487 95.244) (end 120.523 95.244) (width 0.6) (layer F.Cu) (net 2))
 (segment (start 120.523 97.244) (end 120.523 103.044) (width 0.6) (layer F.Cu) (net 2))
 (segment (start 160.51 103.044) (end 160.51 101.044) (width 0.6) (layer F.Cu) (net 2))
 (segment (start 161.2613 101.044) (end 160.51 101.044) (width 0.6) (layer F.Cu) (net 2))
 (segment (start 161.2613 101.044) (end 163.062 101.044) (width 0.6) (layer F.Cu) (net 2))
 (segment (start 163.062 103.044) (end 163.062 101.044) (width 0.6) (layer F.Cu) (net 2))
 (segment (start 160.51 97.244) (end 160.51 99.244) (width 0.6) (layer F.Cu) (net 2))
 (segment (start 157.3368 106.7692) (end 155.262 108.844) (width 0.6) (layer F.Cu) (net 2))
 (segment (start 167.783 108.668) (end 166.721 108.668) (width 0.6) (layer F.Cu) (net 2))
 (segment (start 164.8222 106.7692) (end 157.3368 106.7692) (width 0.6) (layer F.Cu) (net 2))
 (segment (start 166.721 108.668) (end 164.8222 106.7692) (width 0.6) (layer F.Cu) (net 2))
 (segment (start 123.45 97.207) (end 123.446 97.203) (width 0.6) (layer B.Cu) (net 2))
 (segment (start 154.826 109.28) (end 130.28 109.28) (width 0.6) (layer B.Cu) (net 2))
 (segment (start 130.28 109.28) (end 126 105) (width 0.6) (layer B.Cu) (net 2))
 (segment (start 126 103) (end 123.45 100.45) (width 0.6) (layer B.Cu) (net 2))
 (segment (start 155.262 108.844) (end 154.826 109.28) (width 0.6) (layer B.Cu) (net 2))
 (segment (start 126 105) (end 126 103) (width 0.6) (layer B.Cu) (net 2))
 (segment (start 123.45 100.45) (end 123.45 97.207) (width 0.6) (layer B.Cu) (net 2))
 (segment (start 167.766 95.03) (end 172.88 100.144) (width 0.6) (layer F.Cu) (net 2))
 (segment (start 163.062 97.994) (end 166.026 95.03) (width 0.6) (layer F.Cu) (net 2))
 (segment (start 166.026 95.03) (end 167.766 95.03) (width 0.6) (layer F.Cu) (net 2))
 (segment (start 172.1896 105.5904) (end 158.5156 105.5904) (width 0.6) (layer B.Cu) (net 2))
 (segment (start 158.5156 105.5904) (end 155.262 108.844) (width 0.6) (layer B.Cu) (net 2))
 (segment (start 172.88 100.144) (end 172.88 104.9) (width 0.6) (layer B.Cu) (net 2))
 (segment (start 172.88 104.9) (end 172.1896 105.5904) (width 0.6) (layer B.Cu) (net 2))
 (segment (start 183.023 101.048) (end 181.573 101.048) (width 0.6) (layer B.Cu) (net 10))
 (segment (start 176.73 100.14) (end 180.665 100.14) (width 0.6) (layer B.Cu) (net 10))
 (segment (start 180.665 100.14) (end 181.573 101.048) (width 0.6) (layer B.Cu) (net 10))
 (segment (start 176.686758 100.14) (end 176.73 100.14) (width 0.6) (layer F.Cu) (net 10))
 (segment (start 173.699 103.127758) (end 176.686758 100.14) (width 0.6) (layer F.Cu) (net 10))
 (segment (start 172.614 104.111) (end 173.699 104.111) (width 0.6) (layer F.Cu) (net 10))
 (segment (start 173.699 104.111) (end 173.699 103.127758) (width 0.6) (layer F.Cu) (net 10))
 (segment (start 170.346294 100.150294) (end 170.34 100.144) (width 0.6) (layer F.Cu) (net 11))
 (segment (start 170.704 104.111) (end 170.704 102.761) (width 0.6) (layer F.Cu) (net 11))
 (segment (start 170.346294 102.403294) (end 170.346294 100.150294) (width 0.6) (layer F.Cu) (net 11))
 (segment (start 170.704 102.761) (end 170.346294 102.403294) (width 0.6) (layer F.Cu) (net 11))
 (via (at 164.32 107.57) (size 0.6) (drill 0.3) (layers F.Cu B.Cu) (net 3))
 (segment (start 158.6365 107.5695) (end 164.327 107.5695) (width 0.6) (layer F.Cu) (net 3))
 (segment (start 157.362 108.844) (end 158.6365 107.5695) (width 0.6) (layer F.Cu) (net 3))
 (segment (start 164.6607 107.2293) (end 164.32 107.57) (width 0.6) (layer B.Cu) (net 3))
 (segment (start 177.943 108.668) (end 176.5043 107.2293) (width 0.6) (layer B.Cu) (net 3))
 (segment (start 176.5043 107.2293) (end 164.6607 107.2293) (width 0.6) (layer B.Cu) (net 3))
 (segment (start 180.483 108.668) (end 178.244 106.429) (width 0.6) (layer B.Cu) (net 1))
 (segment (start 178.244 106.429) (end 161.877 106.429) (width 0.6) (layer B.Cu) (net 1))
 (segment (start 161.877 106.429) (end 159.462 108.844) (width 0.6) (layer B.Cu) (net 1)))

